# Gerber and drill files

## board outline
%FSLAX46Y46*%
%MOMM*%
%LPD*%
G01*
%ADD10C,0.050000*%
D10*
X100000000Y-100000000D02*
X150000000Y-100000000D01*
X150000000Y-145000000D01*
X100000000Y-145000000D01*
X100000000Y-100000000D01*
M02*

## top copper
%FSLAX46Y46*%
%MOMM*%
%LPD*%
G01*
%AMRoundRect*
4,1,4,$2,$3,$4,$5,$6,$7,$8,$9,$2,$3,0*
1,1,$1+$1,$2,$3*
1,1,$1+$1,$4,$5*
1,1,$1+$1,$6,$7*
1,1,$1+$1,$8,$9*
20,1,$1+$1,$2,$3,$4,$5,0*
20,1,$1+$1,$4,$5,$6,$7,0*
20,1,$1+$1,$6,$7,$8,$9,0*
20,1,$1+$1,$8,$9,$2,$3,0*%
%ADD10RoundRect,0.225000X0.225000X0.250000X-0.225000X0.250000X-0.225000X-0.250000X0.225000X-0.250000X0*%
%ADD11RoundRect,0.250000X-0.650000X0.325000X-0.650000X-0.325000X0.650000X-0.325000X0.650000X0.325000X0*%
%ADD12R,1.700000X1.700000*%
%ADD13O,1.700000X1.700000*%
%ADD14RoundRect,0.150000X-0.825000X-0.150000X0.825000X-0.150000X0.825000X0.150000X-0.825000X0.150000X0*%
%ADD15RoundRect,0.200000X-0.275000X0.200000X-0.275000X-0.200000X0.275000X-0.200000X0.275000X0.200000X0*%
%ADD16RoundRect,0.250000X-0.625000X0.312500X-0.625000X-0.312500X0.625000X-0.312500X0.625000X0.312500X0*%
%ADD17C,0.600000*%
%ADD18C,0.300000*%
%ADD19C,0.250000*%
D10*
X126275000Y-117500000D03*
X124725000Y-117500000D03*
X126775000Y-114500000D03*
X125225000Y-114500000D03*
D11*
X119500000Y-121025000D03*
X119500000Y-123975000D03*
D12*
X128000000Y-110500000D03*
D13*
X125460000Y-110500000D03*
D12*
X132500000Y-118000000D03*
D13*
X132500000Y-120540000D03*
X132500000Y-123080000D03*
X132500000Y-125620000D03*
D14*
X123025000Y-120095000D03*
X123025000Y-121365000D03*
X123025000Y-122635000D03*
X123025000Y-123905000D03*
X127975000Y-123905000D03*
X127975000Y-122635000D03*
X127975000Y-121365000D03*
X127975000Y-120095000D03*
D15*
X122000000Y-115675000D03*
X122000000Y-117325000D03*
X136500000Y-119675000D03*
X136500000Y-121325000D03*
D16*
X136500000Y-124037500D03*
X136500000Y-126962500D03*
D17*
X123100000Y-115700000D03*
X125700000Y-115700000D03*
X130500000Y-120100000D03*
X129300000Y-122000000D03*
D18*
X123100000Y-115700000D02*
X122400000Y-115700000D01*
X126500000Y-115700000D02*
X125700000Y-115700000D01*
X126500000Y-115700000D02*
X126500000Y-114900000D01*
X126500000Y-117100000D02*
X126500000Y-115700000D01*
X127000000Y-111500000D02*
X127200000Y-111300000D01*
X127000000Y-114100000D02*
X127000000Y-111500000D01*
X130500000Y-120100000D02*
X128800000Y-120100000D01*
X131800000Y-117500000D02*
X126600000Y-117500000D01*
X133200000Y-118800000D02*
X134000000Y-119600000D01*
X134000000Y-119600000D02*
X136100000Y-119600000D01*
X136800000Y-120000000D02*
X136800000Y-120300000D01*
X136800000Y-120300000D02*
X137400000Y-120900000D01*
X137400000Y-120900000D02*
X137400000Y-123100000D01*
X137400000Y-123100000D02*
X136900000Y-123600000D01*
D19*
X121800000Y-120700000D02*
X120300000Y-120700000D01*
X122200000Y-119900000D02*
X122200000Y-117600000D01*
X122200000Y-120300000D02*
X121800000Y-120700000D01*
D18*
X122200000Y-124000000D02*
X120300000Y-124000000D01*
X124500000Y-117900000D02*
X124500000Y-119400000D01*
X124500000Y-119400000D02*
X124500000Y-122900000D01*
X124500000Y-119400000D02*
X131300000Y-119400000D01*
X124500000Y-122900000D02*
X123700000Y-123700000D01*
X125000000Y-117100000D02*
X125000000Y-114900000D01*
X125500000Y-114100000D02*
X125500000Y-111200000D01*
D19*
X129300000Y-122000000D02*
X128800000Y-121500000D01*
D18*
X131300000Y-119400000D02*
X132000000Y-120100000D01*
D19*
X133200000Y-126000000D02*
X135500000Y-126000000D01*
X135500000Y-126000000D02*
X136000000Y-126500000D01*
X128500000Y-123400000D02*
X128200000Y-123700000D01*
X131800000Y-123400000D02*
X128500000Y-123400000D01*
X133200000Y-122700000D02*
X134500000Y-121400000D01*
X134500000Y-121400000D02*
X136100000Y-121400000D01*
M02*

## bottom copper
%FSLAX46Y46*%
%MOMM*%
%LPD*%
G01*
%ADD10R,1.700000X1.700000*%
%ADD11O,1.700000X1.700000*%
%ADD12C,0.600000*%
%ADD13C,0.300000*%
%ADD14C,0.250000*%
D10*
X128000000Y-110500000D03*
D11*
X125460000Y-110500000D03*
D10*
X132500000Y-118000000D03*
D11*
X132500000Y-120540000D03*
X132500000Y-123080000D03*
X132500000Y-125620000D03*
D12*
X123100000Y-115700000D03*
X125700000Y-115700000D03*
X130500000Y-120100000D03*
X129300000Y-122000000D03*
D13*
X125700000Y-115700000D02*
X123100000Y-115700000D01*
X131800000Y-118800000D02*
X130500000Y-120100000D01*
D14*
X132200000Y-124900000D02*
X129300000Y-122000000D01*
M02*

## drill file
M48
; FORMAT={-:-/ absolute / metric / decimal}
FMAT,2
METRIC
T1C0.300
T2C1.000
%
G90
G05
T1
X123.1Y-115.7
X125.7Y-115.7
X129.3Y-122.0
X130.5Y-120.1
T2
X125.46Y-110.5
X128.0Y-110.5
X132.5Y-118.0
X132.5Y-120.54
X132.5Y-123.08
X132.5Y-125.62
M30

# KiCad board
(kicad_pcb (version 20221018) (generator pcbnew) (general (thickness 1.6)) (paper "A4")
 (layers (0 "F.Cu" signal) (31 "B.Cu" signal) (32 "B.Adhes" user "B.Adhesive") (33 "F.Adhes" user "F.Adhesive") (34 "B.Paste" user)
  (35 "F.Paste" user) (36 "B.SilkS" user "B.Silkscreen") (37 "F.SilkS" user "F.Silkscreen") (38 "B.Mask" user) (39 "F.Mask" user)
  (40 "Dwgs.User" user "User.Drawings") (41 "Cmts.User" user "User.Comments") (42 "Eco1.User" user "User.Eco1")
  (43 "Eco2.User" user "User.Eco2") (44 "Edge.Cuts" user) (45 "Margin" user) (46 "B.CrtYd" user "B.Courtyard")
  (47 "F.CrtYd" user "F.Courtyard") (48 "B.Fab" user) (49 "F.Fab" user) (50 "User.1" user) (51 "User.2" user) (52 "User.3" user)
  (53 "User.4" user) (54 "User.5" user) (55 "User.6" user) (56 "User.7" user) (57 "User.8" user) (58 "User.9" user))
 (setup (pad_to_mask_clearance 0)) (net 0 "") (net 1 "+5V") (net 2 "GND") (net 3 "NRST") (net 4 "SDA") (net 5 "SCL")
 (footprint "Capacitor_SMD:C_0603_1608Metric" (layer "F.Cu") (at 125.5 117.5 180)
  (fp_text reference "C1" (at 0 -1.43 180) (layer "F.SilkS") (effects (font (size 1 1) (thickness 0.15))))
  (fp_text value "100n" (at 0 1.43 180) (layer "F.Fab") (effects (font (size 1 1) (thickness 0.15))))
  (pad "1" smd roundrect (at -0.775 0 180) (size 0.9 0.95) (layers "F.Cu" "F.Paste" "F.Mask") (roundrect_rratio 0.25) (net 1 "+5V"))
  (pad "2" smd roundrect (at 0.775 0 180) (size 0.9 0.95) (layers "F.Cu" "F.Paste" "F.Mask") (roundrect_rratio 0.25) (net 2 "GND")))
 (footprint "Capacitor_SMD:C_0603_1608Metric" (layer "F.Cu") (at 126 114.5 180)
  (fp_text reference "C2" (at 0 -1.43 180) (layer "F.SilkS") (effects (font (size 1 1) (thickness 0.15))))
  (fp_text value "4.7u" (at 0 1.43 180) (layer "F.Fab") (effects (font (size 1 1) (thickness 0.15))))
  (pad "1" smd roundrect (at -0.775 0 180) (size 0.9 0.95) (layers "F.Cu" "F.Paste" "F.Mask") (roundrect_rratio 0.25) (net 1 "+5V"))
  (pad "2" smd roundrect (at 0.775 0 180) (size 0.9 0.95) (layers "F.Cu" "F.Paste" "F.Mask") (roundrect_rratio 0.25) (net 2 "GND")))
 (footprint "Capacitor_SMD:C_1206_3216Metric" (layer "F.Cu") (at 119.5 122.5 -90)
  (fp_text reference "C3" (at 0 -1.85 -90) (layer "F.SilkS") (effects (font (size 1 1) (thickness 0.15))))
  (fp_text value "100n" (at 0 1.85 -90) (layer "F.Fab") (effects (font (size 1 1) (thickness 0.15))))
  (pad "1" smd roundrect (at -1.475 0 270) (size 1.15 1.8) (layers "F.Cu" "F.Paste" "F.Mask") (roundrect_rratio 0.217391) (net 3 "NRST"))
  (pad "2" smd roundrect (at 1.475 0 270) (size 1.15 1.8) (layers "F.Cu" "F.Paste" "F.Mask") (roundrect_rratio 0.217391) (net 2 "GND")))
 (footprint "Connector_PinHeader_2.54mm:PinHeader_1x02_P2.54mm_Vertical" (layer "F.Cu") (at 128 110.5 -90)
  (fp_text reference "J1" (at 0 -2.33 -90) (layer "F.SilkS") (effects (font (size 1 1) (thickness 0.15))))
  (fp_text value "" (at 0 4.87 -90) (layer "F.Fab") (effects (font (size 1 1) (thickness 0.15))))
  (pad "1" thru_hole rect (at 0 0 270) (size 1.7 1.7) (drill 1) (layers "*.Cu" "*.Mask") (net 1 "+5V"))
  (pad "2" thru_hole oval (at 0 2.54 270) (size 1.7 1.7) (drill 1) (layers "*.Cu" "*.Mask") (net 2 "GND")))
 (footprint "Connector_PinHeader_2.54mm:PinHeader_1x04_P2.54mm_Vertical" (layer "F.Cu") (at 132.5 118)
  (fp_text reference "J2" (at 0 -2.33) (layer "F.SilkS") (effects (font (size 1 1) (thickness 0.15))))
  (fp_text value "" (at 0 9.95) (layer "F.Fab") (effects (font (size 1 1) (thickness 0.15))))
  (pad "1" thru_hole rect (at 0 0) (size 1.7 1.7) (drill 1) (layers "*.Cu" "*.Mask") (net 1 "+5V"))
  (pad "2" thru_hole oval (at 0 2.54) (size 1.7 1.7) (drill 1) (layers "*.Cu" "*.Mask") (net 2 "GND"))
  (pad "3" thru_hole oval (at 0 5.08) (size 1.7 1.7) (drill 1) (layers "*.Cu" "*.Mask") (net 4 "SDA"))
  (pad "4" thru_hole oval (at 0 7.62) (size 1.7 1.7) (drill 1) (layers "*.Cu" "*.Mask") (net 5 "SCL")))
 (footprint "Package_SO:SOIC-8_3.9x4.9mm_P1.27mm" (layer "F.Cu") (at 125.5 122)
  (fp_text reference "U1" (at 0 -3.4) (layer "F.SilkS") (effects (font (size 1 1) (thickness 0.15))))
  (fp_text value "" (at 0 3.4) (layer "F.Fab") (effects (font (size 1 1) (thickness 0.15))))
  (pad "1" smd roundrect (at -2.475 -1.905) (size 1.95 0.6) (layers "F.Cu" "F.Paste" "F.Mask") (roundrect_rratio 0.25) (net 3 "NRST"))
  (pad "2" smd roundrect (at -2.475 -0.635) (size 1.95 0.6) (layers "F.Cu" "F.Paste" "F.Mask") (roundrect_rratio 0.25))
  (pad "3" smd roundrect (at -2.475 0.635) (size 1.95 0.6) (layers "F.Cu" "F.Paste" "F.Mask") (roundrect_rratio 0.25))
  (pad "4" smd roundrect (at -2.475 1.905) (size 1.95 0.6) (layers "F.Cu" "F.Paste" "F.Mask") (roundrect_rratio 0.25) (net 2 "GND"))
  (pad "5" smd roundrect (at 2.475 1.905) (size 1.95 0.6) (layers "F.Cu" "F.Paste" "F.Mask") (roundrect_rratio 0.25) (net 4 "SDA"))
  (pad "6" smd roundrect (at 2.475 0.635) (size 1.95 0.6) (layers "F.Cu" "F.Paste" "F.Mask") (roundrect_rratio 0.25))
  (pad "7" smd roundrect (at 2.475 -0.635) (size 1.95 0.6) (layers "F.Cu" "F.Paste" "F.Mask") (roundrect_rratio 0.25) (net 5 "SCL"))
  (pad "8" smd roundrect (at 2.475 -1.905) (size 1.95 0.6) (layers "F.Cu" "F.Paste" "F.Mask") (roundrect_rratio 0.25) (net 1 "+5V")))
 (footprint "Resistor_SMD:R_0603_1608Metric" (layer "F.Cu") (at 122 116.5 -90)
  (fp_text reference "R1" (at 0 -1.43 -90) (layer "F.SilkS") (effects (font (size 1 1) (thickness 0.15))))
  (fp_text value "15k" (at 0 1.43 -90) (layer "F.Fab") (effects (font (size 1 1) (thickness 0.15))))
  (pad "1" smd roundrect (at -0.825 0 270) (size 0.8 0.95) (layers "F.Cu" "F.Paste" "F.Mask") (roundrect_rratio 0.25) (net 1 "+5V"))
  (pad "2" smd roundrect (at 0.825 0 270) (size 0.8 0.95) (layers "F.Cu" "F.Paste" "F.Mask") (roundrect_rratio 0.25) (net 3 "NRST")))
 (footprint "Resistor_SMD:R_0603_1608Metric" (layer "F.Cu") (at 136.5 120.5 -90)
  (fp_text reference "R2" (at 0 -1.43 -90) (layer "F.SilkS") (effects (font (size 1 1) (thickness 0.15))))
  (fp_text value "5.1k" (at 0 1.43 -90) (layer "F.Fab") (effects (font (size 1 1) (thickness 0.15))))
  (pad "1" smd roundrect (at -0.825 0 270) (size 0.8 0.95) (layers "F.Cu" "F.Paste" "F.Mask") (roundrect_rratio 0.25) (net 1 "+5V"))
  (pad "2" smd roundrect (at 0.825 0 270) (size 0.8 0.95) (layers "F.Cu" "F.Paste" "F.Mask") (roundrect_rratio 0.25) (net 4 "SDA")))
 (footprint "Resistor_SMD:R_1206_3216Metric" (layer "F.Cu") (at 136.5 125.5 -90)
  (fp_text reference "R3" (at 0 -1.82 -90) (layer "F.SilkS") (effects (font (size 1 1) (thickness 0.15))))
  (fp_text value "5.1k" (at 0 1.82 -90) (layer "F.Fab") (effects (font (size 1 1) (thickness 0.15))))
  (pad "1" smd roundrect (at -1.4625 0 270) (size 1.125 1.75) (layers "F.Cu" "F.Paste" "F.Mask") (roundrect_rratio 0.222222) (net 1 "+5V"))
  (pad "2" smd roundrect (at 1.4625 0 270) (size 1.125 1.75) (layers "F.Cu" "F.Paste" "F.Mask") (roundrect_rratio 0.222222) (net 5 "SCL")))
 (gr_rect (start 100 100) (end 150 145) (stroke (width 0.05) (type default)) (fill none) (layer "Edge.Cuts"))
 (segment (start 123.1 115.7) (end 122.4 115.7) (width 0.3) (layer "F.Cu") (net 1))
 (segment (start 126.5 115.7) (end 125.7 115.7) (width 0.3) (layer "F.Cu") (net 1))
 (segment (start 126.5 115.7) (end 126.5 114.9) (width 0.3) (layer "F.Cu") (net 1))
 (segment (start 126.5 117.1) (end 126.5 115.7) (width 0.3) (layer "F.Cu") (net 1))
 (segment (start 127 111.5) (end 127.2 111.3) (width 0.3) (layer "F.Cu") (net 1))
 (segment (start 127 114.1) (end 127 111.5) (width 0.3) (layer "F.Cu") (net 1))
 (segment (start 130.5 120.1) (end 128.8 120.1) (width 0.3) (layer "F.Cu") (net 1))
 (segment (start 131.8 117.5) (end 126.6 117.5) (width 0.3) (layer "F.Cu") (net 1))
 (segment (start 133.2 118.8) (end 134 119.6) (width 0.3) (layer "F.Cu") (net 1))
 (segment (start 134 119.6) (end 136.1 119.6) (width 0.3) (layer "F.Cu") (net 1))
 (segment (start 136.8 120) (end 136.8 120.3) (width 0.3) (layer "F.Cu") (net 1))
 (segment (start 136.8 120.3) (end 137.4 120.9) (width 0.3) (layer "F.Cu") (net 1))
 (segment (start 137.4 120.9) (end 137.4 123.1) (width 0.3) (layer "F.Cu") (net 1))
 (segment (start 137.4 123.1) (end 136.9 123.6) (width 0.3) (layer "F.Cu") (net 1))
 (via (at 123.1 115.7) (size 0.6) (drill 0.3) (layers "F.Cu" "B.Cu") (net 1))
 (via (at 125.7 115.7) (size 0.6) (drill 0.3) (layers "F.Cu" "B.Cu") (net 1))
 (via (at 130.5 120.1) (size 0.6) (drill 0.3) (layers "F.Cu" "B.Cu") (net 1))
 (segment (start 121.8 120.7) (end 120.3 120.7) (width 0.25) (layer "F.Cu") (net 3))
 (segment (start 122.2 119.9) (end 122.2 117.6) (width 0.25) (layer "F.Cu") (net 3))
 (segment (start 122.2 120.3) (end 121.8 120.7) (width 0.25) (layer "F.Cu") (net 3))
 (segment (start 122.2 124) (end 120.3 124) (width 0.3) (layer "F.Cu") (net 2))
 (segment (start 124.5 117.9) (end 124.5 119.4) (width 0.3) (layer "F.Cu") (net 2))
 (segment (start 124.5 119.4) (end 124.5 122.9) (width 0.3) (layer "F.Cu") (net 2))
 (segment (start 124.5 119.4) (end 131.3 119.4) (width 0.3) (layer "F.Cu") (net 2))
 (segment (start 124.5 122.9) (end 123.7 123.7) (width 0.3) (layer "F.Cu") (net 2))
 (segment (start 125 117.1) (end 125 114.9) (width 0.3) (layer "F.Cu") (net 2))
 (segment (start 125.5 114.1) (end 125.5 111.2) (width 0.3) (layer "F.Cu") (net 2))
 (segment (start 125.7 115.7) (end 123.1 115.7) (width 0.3) (layer "B.Cu") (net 1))
 (segment (start 129.3 122) (end 128.8 121.5) (width 0.25) (layer "F.Cu") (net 5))
 (segment (start 131.3 119.4) (end 132 120.1) (width 0.3) (layer "F.Cu") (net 2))
 (segment (start 131.8 118.8) (end 130.5 120.1) (width 0.3) (layer "B.Cu") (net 1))
 (segment (start 133.2 126) (end 135.5 126) (width 0.25) (layer "F.Cu") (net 5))
 (segment (start 135.5 126) (end 136 126.5) (width 0.25) (layer "F.Cu") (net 5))
 (via (at 129.3 122) (size 0.6) (drill 0.3) (layers "F.Cu" "B.Cu") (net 5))
 (segment (start 128.5 123.4) (end 128.2 123.7) (width 0.25) (layer "F.Cu") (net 4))
 (segment (start 131.8 123.4) (end 128.5 123.4) (width 0.25) (layer "F.Cu") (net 4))
 (segment (start 132.2 124.9) (end 129.3 122) (width 0.25) (layer "B.Cu") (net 5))
 (segment (start 133.2 122.7) (end 134.5 121.4) (width 0.25) (layer "F.Cu") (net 4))
 (segment (start 134.5 121.4) (end 136.1 121.4) (width 0.25) (layer "F.Cu") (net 4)))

